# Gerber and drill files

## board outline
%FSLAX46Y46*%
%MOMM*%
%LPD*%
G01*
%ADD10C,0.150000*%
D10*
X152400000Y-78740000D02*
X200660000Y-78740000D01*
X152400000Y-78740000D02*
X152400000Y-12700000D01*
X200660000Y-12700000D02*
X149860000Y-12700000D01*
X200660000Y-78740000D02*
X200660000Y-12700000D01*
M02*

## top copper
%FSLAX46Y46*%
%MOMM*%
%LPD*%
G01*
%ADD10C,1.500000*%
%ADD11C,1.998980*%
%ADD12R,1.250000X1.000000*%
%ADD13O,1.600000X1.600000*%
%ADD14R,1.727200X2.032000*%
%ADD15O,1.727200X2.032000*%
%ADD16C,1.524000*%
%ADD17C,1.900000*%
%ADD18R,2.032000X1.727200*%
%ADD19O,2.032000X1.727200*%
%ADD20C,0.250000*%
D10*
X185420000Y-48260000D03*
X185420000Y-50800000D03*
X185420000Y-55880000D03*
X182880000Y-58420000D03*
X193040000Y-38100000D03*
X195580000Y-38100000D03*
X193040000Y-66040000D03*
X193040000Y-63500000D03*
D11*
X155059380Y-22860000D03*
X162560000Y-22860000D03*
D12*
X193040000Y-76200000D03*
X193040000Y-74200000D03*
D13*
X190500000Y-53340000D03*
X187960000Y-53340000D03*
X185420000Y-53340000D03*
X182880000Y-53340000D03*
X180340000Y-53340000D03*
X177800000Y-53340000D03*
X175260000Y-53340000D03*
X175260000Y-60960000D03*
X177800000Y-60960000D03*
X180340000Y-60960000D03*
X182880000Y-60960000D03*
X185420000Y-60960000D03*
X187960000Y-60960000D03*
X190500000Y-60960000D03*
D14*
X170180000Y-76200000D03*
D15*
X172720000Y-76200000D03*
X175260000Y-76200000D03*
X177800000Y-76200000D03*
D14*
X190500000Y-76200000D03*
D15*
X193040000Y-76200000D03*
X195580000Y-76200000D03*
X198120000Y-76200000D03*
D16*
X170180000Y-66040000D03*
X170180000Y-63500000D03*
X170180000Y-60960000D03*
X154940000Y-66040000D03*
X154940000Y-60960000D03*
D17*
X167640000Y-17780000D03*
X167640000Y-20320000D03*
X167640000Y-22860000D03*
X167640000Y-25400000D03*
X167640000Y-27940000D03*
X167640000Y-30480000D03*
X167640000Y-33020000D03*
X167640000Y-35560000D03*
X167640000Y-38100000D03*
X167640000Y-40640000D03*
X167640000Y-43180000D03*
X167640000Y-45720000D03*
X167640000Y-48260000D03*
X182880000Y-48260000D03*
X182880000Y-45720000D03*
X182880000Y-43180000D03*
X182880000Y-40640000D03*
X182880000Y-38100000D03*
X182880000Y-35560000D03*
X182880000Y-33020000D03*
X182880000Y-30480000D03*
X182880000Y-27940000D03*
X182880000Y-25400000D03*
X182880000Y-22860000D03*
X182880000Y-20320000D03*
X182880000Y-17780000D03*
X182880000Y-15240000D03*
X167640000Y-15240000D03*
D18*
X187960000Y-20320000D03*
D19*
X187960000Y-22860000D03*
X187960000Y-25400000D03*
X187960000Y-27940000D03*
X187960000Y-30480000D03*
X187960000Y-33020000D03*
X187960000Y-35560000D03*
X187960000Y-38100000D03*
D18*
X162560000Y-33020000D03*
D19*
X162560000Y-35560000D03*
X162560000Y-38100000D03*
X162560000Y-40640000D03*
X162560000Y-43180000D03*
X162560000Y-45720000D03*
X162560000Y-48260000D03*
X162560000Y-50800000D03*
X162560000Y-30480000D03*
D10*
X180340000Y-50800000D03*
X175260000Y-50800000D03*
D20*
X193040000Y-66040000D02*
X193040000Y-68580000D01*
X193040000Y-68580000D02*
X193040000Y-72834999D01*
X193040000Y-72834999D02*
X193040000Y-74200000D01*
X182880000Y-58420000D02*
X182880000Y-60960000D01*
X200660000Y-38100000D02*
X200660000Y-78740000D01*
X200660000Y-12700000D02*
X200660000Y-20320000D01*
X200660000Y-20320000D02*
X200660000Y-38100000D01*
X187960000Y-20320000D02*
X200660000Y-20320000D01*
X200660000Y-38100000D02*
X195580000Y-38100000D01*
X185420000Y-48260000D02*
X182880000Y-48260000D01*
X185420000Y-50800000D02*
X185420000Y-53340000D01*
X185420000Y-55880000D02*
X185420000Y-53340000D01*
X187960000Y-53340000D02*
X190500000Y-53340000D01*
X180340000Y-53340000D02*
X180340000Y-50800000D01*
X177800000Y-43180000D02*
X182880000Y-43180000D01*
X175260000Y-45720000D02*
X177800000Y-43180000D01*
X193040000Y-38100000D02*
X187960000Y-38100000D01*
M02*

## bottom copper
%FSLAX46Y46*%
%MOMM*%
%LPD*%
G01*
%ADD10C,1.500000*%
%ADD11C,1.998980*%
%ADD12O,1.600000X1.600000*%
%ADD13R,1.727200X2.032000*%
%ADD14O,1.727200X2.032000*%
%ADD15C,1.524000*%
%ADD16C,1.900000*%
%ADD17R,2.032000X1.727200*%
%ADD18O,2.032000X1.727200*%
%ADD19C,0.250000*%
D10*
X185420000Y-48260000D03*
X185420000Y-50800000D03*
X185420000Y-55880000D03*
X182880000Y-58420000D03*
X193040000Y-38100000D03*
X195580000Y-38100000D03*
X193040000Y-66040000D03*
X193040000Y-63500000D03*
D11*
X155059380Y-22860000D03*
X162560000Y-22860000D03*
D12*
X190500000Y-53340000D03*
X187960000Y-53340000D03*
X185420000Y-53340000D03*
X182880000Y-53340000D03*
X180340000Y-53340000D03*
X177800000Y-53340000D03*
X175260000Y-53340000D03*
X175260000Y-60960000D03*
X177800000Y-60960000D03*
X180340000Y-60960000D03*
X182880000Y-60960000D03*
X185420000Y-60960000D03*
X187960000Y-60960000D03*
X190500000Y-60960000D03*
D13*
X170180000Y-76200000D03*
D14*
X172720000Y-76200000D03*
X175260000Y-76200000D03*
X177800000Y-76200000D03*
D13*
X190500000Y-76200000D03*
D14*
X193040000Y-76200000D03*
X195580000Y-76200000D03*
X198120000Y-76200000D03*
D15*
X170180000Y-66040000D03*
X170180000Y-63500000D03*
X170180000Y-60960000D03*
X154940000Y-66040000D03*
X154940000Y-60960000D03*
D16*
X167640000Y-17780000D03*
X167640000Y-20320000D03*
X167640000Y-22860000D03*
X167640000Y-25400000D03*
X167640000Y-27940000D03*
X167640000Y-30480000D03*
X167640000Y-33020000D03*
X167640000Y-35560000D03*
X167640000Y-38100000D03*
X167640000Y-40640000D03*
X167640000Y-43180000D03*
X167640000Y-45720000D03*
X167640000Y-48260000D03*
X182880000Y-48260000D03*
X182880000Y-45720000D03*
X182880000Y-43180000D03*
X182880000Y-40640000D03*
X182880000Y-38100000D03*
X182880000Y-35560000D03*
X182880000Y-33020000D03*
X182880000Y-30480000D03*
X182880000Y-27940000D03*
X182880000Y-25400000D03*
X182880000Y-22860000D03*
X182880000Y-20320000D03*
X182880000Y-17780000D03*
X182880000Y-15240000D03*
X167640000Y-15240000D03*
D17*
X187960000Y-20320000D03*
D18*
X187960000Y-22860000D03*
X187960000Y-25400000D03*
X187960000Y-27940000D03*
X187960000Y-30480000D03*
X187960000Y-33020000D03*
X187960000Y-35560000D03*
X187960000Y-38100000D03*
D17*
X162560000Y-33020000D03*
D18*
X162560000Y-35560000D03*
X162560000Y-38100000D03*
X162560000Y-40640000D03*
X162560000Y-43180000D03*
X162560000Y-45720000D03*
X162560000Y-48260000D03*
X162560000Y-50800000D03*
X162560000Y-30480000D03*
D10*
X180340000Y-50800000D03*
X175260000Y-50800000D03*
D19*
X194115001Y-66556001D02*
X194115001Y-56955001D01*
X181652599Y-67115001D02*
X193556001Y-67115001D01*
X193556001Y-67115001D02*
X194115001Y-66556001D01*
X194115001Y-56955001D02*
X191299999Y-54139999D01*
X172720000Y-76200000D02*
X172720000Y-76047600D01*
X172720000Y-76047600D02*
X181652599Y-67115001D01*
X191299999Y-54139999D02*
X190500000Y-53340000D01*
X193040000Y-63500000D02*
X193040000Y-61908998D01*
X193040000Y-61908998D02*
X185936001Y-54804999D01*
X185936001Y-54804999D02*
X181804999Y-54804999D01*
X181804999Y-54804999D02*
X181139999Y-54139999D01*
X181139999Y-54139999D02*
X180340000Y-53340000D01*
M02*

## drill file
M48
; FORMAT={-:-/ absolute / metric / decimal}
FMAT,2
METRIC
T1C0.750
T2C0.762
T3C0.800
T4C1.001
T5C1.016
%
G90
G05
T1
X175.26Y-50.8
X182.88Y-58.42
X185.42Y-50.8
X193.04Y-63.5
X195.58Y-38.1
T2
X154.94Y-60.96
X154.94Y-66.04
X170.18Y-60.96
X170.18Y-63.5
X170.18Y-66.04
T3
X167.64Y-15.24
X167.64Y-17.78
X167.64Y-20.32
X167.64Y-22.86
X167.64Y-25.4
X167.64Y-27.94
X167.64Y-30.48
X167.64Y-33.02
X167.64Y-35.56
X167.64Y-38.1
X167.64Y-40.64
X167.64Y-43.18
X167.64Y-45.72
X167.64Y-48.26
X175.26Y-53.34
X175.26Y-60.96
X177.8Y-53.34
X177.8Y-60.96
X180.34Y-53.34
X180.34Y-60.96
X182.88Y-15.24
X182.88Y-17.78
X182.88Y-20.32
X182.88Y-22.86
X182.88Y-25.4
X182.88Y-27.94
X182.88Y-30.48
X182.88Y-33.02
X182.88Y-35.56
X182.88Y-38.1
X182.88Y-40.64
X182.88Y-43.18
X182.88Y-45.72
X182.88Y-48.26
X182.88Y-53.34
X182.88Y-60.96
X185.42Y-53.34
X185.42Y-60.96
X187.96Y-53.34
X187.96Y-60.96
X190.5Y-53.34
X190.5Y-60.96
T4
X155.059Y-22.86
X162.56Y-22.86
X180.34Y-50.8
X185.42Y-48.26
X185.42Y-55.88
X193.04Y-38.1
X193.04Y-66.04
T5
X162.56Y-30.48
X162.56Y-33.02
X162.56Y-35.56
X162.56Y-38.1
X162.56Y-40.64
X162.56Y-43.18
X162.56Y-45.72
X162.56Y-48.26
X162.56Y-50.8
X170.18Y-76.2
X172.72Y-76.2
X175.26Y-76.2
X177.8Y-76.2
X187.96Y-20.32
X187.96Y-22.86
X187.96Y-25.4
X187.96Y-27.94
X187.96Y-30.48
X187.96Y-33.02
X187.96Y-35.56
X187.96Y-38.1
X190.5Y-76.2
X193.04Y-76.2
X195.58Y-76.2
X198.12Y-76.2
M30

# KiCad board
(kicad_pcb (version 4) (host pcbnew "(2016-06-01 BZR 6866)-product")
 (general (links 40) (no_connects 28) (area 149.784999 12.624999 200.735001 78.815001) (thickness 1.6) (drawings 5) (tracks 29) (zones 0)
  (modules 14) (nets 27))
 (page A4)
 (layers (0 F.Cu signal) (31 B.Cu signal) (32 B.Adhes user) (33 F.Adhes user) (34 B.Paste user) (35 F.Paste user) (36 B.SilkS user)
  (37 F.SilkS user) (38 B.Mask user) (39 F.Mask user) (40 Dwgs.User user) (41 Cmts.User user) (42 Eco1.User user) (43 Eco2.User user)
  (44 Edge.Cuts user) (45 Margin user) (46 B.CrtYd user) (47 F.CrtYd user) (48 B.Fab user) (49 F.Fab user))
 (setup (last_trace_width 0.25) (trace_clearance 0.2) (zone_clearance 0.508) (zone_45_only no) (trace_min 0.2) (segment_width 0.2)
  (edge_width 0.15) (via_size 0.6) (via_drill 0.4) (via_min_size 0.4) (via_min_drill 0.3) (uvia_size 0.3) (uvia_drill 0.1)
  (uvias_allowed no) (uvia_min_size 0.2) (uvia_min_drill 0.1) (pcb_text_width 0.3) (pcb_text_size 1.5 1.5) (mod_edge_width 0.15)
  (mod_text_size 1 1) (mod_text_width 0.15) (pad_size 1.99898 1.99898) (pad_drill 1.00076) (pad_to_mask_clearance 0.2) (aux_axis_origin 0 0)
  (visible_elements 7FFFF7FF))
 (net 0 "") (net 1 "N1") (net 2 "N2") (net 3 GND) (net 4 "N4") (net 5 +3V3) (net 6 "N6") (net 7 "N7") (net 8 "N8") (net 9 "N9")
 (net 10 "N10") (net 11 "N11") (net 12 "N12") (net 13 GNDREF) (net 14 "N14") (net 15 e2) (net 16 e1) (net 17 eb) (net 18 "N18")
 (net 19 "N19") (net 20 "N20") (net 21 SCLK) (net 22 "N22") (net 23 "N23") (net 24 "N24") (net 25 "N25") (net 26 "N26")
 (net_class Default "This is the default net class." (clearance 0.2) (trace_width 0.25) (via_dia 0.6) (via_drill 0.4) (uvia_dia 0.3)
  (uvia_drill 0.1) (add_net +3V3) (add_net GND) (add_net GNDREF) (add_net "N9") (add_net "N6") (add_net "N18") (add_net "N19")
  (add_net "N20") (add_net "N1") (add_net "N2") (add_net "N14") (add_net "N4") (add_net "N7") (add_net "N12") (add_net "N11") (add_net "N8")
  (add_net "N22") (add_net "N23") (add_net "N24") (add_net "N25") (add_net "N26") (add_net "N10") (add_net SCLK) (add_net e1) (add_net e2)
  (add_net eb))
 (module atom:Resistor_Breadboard (layer F.Cu) (at 185.42 50.8 270)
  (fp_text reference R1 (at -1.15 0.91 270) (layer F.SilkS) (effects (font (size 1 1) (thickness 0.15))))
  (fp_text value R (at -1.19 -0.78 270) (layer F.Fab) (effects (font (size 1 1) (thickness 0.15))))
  (pad 1 thru_hole circle (at -2.54 0 270) (size 1.5 1.5) (drill 1.00076) (layers *.Cu *.SilkS *.Mask) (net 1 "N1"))
  (pad 2 thru_hole circle (at 0 0 270) (size 1.5 1.5) (drill 0.75) (layers *.Cu *.SilkS *.Mask) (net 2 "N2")))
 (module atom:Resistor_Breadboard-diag (layer F.Cu) (at 182.88 58.42 180)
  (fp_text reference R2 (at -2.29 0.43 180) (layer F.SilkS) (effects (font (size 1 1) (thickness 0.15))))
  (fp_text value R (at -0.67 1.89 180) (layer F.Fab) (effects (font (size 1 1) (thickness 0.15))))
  (pad 1 thru_hole circle (at -2.54 2.54 180) (size 1.5 1.5) (drill 1.00076) (layers *.Cu *.SilkS *.Mask) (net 2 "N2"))
  (pad 2 thru_hole circle (at 0 0 180) (size 1.5 1.5) (drill 0.75) (layers *.Cu *.SilkS *.Mask) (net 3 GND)))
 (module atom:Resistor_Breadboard (layer F.Cu) (at 195.58 38.1)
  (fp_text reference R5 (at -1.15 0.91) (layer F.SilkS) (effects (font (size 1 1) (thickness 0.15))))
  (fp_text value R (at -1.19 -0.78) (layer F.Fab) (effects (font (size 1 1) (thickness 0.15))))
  (pad 1 thru_hole circle (at -2.54 0) (size 1.5 1.5) (drill 1.00076) (layers *.Cu *.SilkS *.Mask) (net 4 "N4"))
  (pad 2 thru_hole circle (at 0 0) (size 1.5 1.5) (drill 0.75) (layers *.Cu *.SilkS *.Mask) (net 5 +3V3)))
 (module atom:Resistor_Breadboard (layer F.Cu) (at 193.04 63.5 90)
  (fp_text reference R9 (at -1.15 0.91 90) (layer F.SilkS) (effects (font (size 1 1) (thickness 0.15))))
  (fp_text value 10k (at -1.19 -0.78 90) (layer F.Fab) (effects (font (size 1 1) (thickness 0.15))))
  (pad 1 thru_hole circle (at -2.54 0 90) (size 1.5 1.5) (drill 1.00076) (layers *.Cu *.SilkS *.Mask) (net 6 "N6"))
  (pad 2 thru_hole circle (at 0 0 90) (size 1.5 1.5) (drill 0.75) (layers *.Cu *.SilkS *.Mask) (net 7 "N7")))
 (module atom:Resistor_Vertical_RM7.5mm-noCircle (layer F.Cu) (at 158.80842 22.86)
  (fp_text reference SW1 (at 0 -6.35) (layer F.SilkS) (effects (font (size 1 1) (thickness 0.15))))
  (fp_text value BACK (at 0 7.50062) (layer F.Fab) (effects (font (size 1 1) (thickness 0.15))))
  (pad 1 thru_hole circle (at -3.74904 0) (size 1.99898 1.99898) (drill 1.00076) (layers *.Cu *.SilkS *.Mask) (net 3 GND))
  (pad 2 thru_hole circle (at 3.75158 0) (size 1.99898 1.99898) (drill 1.00076) (layers *.Cu *.SilkS *.Mask) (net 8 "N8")))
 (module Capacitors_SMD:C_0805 (layer F.Cu) (at 193.04 75.2 90)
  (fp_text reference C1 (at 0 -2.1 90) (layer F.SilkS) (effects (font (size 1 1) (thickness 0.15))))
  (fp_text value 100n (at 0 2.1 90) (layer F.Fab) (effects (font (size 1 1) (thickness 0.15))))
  (pad 1 smd rect (at -1 0 90) (size 1 1.25) (layers F.Cu F.Paste F.Mask) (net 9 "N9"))
  (pad 2 smd rect (at 1 0 90) (size 1 1.25) (layers F.Cu F.Paste F.Mask) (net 6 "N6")))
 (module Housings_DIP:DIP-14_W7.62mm (layer F.Cu) (at 190.5 53.34 270)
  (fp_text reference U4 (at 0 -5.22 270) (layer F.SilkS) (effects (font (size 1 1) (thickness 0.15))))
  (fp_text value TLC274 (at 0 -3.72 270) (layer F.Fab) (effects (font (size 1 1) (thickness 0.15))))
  (pad 1 thru_hole oval (at 0 0 270) (size 1.6 1.6) (drill 0.8) (layers *.Cu *.Mask F.SilkS) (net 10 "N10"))
  (pad 2 thru_hole oval (at 0 2.54 270) (size 1.6 1.6) (drill 0.8) (layers *.Cu *.Mask F.SilkS) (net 10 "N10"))
  (pad 3 thru_hole oval (at 0 5.08 270) (size 1.6 1.6) (drill 0.8) (layers *.Cu *.Mask F.SilkS) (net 2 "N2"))
  (pad 4 thru_hole oval (at 0 7.62 270) (size 1.6 1.6) (drill 0.8) (layers *.Cu *.Mask F.SilkS) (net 5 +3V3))
  (pad 5 thru_hole oval (at 0 10.16 270) (size 1.6 1.6) (drill 0.8) (layers *.Cu *.Mask F.SilkS) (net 7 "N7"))
  (pad 6 thru_hole oval (at 0 12.7 270) (size 1.6 1.6) (drill 0.8) (layers *.Cu *.Mask F.SilkS) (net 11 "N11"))
  (pad 7 thru_hole oval (at 0 15.24 270) (size 1.6 1.6) (drill 0.8) (layers *.Cu *.Mask F.SilkS) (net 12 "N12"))
  (pad 8 thru_hole oval (at 7.62 15.24 270) (size 1.6 1.6) (drill 0.8) (layers *.Cu *.Mask F.SilkS) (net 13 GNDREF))
  (pad 9 thru_hole oval (at 7.62 12.7 270) (size 1.6 1.6) (drill 0.8) (layers *.Cu *.Mask F.SilkS) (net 13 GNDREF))
  (pad 10 thru_hole oval (at 7.62 10.16 270) (size 1.6 1.6) (drill 0.8) (layers *.Cu *.Mask F.SilkS) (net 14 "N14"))
  (pad 11 thru_hole oval (at 7.62 7.62 270) (size 1.6 1.6) (drill 0.8) (layers *.Cu *.Mask F.SilkS) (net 3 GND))
  (pad 12 thru_hole oval (at 7.62 5.08 270) (size 1.6 1.6) (drill 0.8) (layers *.Cu *.Mask F.SilkS))
  (pad 13 thru_hole oval (at 7.62 2.54 270) (size 1.6 1.6) (drill 0.8) (layers *.Cu *.Mask F.SilkS))
  (pad 14 thru_hole oval (at 7.62 0 270) (size 1.6 1.6) (drill 0.8) (layers *.Cu *.Mask F.SilkS)))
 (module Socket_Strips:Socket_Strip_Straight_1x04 (layer F.Cu) (at 170.18 76.2)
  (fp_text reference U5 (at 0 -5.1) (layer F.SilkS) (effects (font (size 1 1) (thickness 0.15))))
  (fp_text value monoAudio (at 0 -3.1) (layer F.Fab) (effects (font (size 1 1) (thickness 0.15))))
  (pad 1 thru_hole rect (at 0 0) (size 1.7272 2.032) (drill 1.016) (layers *.Cu *.Mask F.SilkS) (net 3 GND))
  (pad 2 thru_hole oval (at 2.54 0) (size 1.7272 2.032) (drill 1.016) (layers *.Cu *.Mask F.SilkS) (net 10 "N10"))
  (pad 3 thru_hole oval (at 5.08 0) (size 1.7272 2.032) (drill 1.016) (layers *.Cu *.Mask F.SilkS))
  (pad 4 thru_hole oval (at 7.62 0) (size 1.7272 2.032) (drill 1.016) (layers *.Cu *.Mask F.SilkS)))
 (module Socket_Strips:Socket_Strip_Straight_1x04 (layer F.Cu) (at 190.5 76.2)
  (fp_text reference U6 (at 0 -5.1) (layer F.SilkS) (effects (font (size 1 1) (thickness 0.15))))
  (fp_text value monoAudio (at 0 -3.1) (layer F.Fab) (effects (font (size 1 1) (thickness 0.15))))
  (pad 1 thru_hole rect (at 0 0) (size 1.7272 2.032) (drill 1.016) (layers *.Cu *.Mask F.SilkS) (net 3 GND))
  (pad 2 thru_hole oval (at 2.54 0) (size 1.7272 2.032) (drill 1.016) (layers *.Cu *.Mask F.SilkS) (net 9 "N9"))
  (pad 3 thru_hole oval (at 5.08 0) (size 1.7272 2.032) (drill 1.016) (layers *.Cu *.Mask F.SilkS))
  (pad 4 thru_hole oval (at 7.62 0) (size 1.7272 2.032) (drill 1.016) (layers *.Cu *.Mask F.SilkS)))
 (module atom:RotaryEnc (layer F.Cu) (at 162.56 63.5 180)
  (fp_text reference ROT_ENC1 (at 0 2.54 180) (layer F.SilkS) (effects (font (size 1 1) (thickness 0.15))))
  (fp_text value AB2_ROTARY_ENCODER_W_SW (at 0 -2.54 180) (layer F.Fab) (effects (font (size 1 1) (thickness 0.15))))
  (pad 1 thru_hole circle (at -7.62 -2.54 180) (size 1.524 1.524) (drill 0.762) (layers *.Cu *.Mask F.SilkS) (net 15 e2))
  (pad 2 thru_hole circle (at -7.62 0 180) (size 1.524 1.524) (drill 0.762) (layers *.Cu *.Mask F.SilkS) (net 3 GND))
  (pad 3 thru_hole circle (at -7.62 2.54 180) (size 1.524 1.524) (drill 0.762) (layers *.Cu *.Mask F.SilkS) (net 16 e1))
  (pad 4 thru_hole circle (at 7.62 -2.54 180) (size 1.524 1.524) (drill 0.762) (layers *.Cu *.Mask F.SilkS) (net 3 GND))
  (pad 5 thru_hole circle (at 7.62 2.54 180) (size 1.524 1.524) (drill 0.762) (layers *.Cu *.Mask F.SilkS) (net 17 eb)))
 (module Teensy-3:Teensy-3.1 (layer F.Cu) (at 167.64 17.78 270)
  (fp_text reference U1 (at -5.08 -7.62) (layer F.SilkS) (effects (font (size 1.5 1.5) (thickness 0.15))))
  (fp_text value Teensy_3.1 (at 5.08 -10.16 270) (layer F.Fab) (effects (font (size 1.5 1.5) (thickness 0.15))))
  (pad 0 thru_hole circle (at 0 0 270) (size 1.9 1.9) (drill 0.8) (layers *.Cu *.Mask F.SilkS))
  (pad 1 thru_hole circle (at 2.54 0 270) (size 1.9 1.9) (drill 0.8) (layers *.Cu *.Mask F.SilkS))
  (pad 2 thru_hole circle (at 5.08 0 270) (size 1.9 1.9) (drill 0.8) (layers *.Cu *.Mask F.SilkS) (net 8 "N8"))
  (pad 3 thru_hole circle (at 7.62 0 270) (size 1.9 1.9) (drill 0.8) (layers *.Cu *.Mask F.SilkS))
  (pad 4 thru_hole circle (at 10.16 0 270) (size 1.9 1.9) (drill 0.8) (layers *.Cu *.Mask F.SilkS))
  (pad 5 thru_hole circle (at 12.7 0 270) (size 1.9 1.9) (drill 0.8) (layers *.Cu *.Mask F.SilkS))
  (pad 6 thru_hole circle (at 15.24 0 270) (size 1.9 1.9) (drill 0.8) (layers *.Cu *.Mask F.SilkS) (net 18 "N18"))
  (pad 7 thru_hole circle (at 17.78 0 270) (size 1.9 1.9) (drill 0.8) (layers *.Cu *.Mask F.SilkS) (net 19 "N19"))
  (pad 8 thru_hole circle (at 20.32 0 270) (size 1.9 1.9) (drill 0.8) (layers *.Cu *.Mask F.SilkS))
  (pad 9 thru_hole circle (at 22.86 0 270) (size 1.9 1.9) (drill 0.8) (layers *.Cu *.Mask F.SilkS) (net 16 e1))
  (pad 10 thru_hole circle (at 25.4 0 270) (size 1.9 1.9) (drill 0.8) (layers *.Cu *.Mask F.SilkS) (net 15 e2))
  (pad 11 thru_hole circle (at 27.94 0 270) (size 1.9 1.9) (drill 0.8) (layers *.Cu *.Mask F.SilkS) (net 17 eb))
  (pad 12 thru_hole circle (at 30.48 0 270) (size 1.9 1.9) (drill 0.8) (layers *.Cu *.Mask F.SilkS) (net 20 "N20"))
  (pad 13 thru_hole circle (at 30.48 -15.24 270) (size 1.9 1.9) (drill 0.8) (layers *.Cu *.Mask F.SilkS) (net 1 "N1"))
  (pad 14 thru_hole circle (at 27.94 -15.24 270) (size 1.9 1.9) (drill 0.8) (layers *.Cu *.Mask F.SilkS) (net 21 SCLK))
  (pad 15 thru_hole circle (at 25.4 -15.24 270) (size 1.9 1.9) (drill 0.8) (layers *.Cu *.Mask F.SilkS) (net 12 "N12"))
  (pad 16 thru_hole circle (at 22.86 -15.24 270) (size 1.9 1.9) (drill 0.8) (layers *.Cu *.Mask F.SilkS))
  (pad 17 thru_hole circle (at 20.32 -15.24 270) (size 1.9 1.9) (drill 0.8) (layers *.Cu *.Mask F.SilkS))
  (pad 18 thru_hole circle (at 17.78 -15.24 270) (size 1.9 1.9) (drill 0.8) (layers *.Cu *.Mask F.SilkS) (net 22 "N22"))
  (pad 19 thru_hole circle (at 15.24 -15.24 270) (size 1.9 1.9) (drill 0.8) (layers *.Cu *.Mask F.SilkS) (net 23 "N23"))
  (pad 20 thru_hole circle (at 12.7 -15.24 270) (size 1.9 1.9) (drill 0.8) (layers *.Cu *.Mask F.SilkS) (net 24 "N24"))
  (pad 21 thru_hole circle (at 10.16 -15.24 270) (size 1.9 1.9) (drill 0.8) (layers *.Cu *.Mask F.SilkS) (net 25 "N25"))
  (pad 22 thru_hole circle (at 7.62 -15.24 270) (size 1.9 1.9) (drill 0.8) (layers *.Cu *.Mask F.SilkS) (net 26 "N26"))
  (pad 23 thru_hole circle (at 5.08 -15.24 270) (size 1.9 1.9) (drill 0.8) (layers *.Cu *.Mask F.SilkS))
  (pad 24 thru_hole circle (at 2.54 -15.24 270) (size 1.9 1.9) (drill 0.8) (layers *.Cu *.Mask F.SilkS) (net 5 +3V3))
  (pad 25 thru_hole circle (at 0 -15.24 270) (size 1.9 1.9) (drill 0.8) (layers *.Cu *.Mask F.SilkS))
  (pad 26 thru_hole circle (at -2.54 -15.24 270) (size 1.9 1.9) (drill 0.8) (layers *.Cu *.Mask F.SilkS))
  (pad 27 thru_hole circle (at -2.54 0 270) (size 1.9 1.9) (drill 0.8) (layers *.Cu *.Mask F.SilkS) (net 3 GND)))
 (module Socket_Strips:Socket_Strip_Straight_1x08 (layer F.Cu) (at 187.96 20.32 270)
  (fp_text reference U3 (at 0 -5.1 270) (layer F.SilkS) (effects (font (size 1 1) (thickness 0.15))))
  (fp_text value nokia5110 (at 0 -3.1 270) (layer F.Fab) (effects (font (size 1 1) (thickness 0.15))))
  (pad 1 thru_hole rect (at 0 0 270) (size 1.7272 2.032) (drill 1.016) (layers *.Cu *.Mask F.SilkS) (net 5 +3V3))
  (pad 2 thru_hole oval (at 2.54 0 270) (size 1.7272 2.032) (drill 1.016) (layers *.Cu *.Mask F.SilkS) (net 3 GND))
  (pad 3 thru_hole oval (at 5.08 0 270) (size 1.7272 2.032) (drill 1.016) (layers *.Cu *.Mask F.SilkS) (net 26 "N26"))
  (pad 4 thru_hole oval (at 7.62 0 270) (size 1.7272 2.032) (drill 1.016) (layers *.Cu *.Mask F.SilkS) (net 25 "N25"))
  (pad 5 thru_hole oval (at 10.16 0 270) (size 1.7272 2.032) (drill 1.016) (layers *.Cu *.Mask F.SilkS) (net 24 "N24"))
  (pad 6 thru_hole oval (at 12.7 0 270) (size 1.7272 2.032) (drill 1.016) (layers *.Cu *.Mask F.SilkS) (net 23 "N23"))
  (pad 7 thru_hole oval (at 15.24 0 270) (size 1.7272 2.032) (drill 1.016) (layers *.Cu *.Mask F.SilkS) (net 22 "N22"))
  (pad 8 thru_hole oval (at 17.78 0 270) (size 1.7272 2.032) (drill 1.016) (layers *.Cu *.Mask F.SilkS) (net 4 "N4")))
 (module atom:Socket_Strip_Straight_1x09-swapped (layer F.Cu) (at 162.56 33.02 270)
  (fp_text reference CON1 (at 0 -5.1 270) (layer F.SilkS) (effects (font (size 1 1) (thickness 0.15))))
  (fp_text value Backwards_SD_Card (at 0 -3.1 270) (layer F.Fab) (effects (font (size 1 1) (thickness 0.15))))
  (pad 1 thru_hole rect (at 0 0 270) (size 1.7272 2.032) (drill 1.016) (layers *.Cu *.Mask F.SilkS) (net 18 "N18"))
  (pad 2 thru_hole oval (at 2.54 0 270) (size 1.7272 2.032) (drill 1.016) (layers *.Cu *.Mask F.SilkS) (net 19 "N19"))
  (pad 3 thru_hole oval (at 5.08 0 270) (size 1.7272 2.032) (drill 1.016) (layers *.Cu *.Mask F.SilkS) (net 3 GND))
  (pad 4 thru_hole oval (at 7.62 0 270) (size 1.7272 2.032) (drill 1.016) (layers *.Cu *.Mask F.SilkS) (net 5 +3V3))
  (pad 5 thru_hole oval (at 10.16 0 270) (size 1.7272 2.032) (drill 1.016) (layers *.Cu *.Mask F.SilkS) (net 21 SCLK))
  (pad 6 thru_hole oval (at 12.7 0 270) (size 1.7272 2.032) (drill 1.016) (layers *.Cu *.Mask F.SilkS) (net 3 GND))
  (pad 7 thru_hole oval (at 15.24 0 270) (size 1.7272 2.032) (drill 1.016) (layers *.Cu *.Mask F.SilkS) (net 20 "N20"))
  (pad 8 thru_hole oval (at 17.78 0 270) (size 1.7272 2.032) (drill 1.016) (layers *.Cu *.Mask F.SilkS))
  (pad 9 thru_hole oval (at -2.54 0 270) (size 1.7272 2.032) (drill 1.016) (layers *.Cu *.Mask F.SilkS)))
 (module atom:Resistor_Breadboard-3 (layer F.Cu) (at 177.8 50.8 180)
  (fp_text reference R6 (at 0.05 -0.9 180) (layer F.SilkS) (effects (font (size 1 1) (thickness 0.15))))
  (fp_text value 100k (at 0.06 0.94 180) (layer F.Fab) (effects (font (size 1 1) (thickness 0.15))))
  (pad 1 thru_hole circle (at -2.54 0 180) (size 1.5 1.5) (drill 1.00076) (layers *.Cu *.SilkS *.Mask) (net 7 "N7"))
  (pad 2 thru_hole circle (at 2.54 0 180) (size 1.5 1.5) (drill 0.75) (layers *.Cu *.SilkS *.Mask) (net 12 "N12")))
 (gr_line (start 152.4 78.74) (end 200.66 78.74) (layer Edge.Cuts) (width 0.15))
 (gr_line (start 152.4 78.74) (end 152.4 12.7) (layer Edge.Cuts) (width 0.15))
 (gr_line (start 200.66 12.7) (end 149.86 12.7) (layer Edge.Cuts) (width 0.15))
 (gr_line (start 200.66 78.74) (end 200.66 12.7) (layer Edge.Cuts) (width 0.15))
 (segment (start 193.04 66.04) (end 193.04 68.58) (width 0.25) (layer F.Cu) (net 6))
 (segment (start 193.04 68.58) (end 193.04 72.834999) (width 0.25) (layer F.Cu) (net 6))
 (segment (start 193.04 72.834999) (end 193.04 74.2) (width 0.25) (layer F.Cu) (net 6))
 (segment (start 182.88 58.42) (end 182.88 60.96) (width 0.25) (layer F.Cu) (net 3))
 (segment (start 200.66 38.1) (end 200.66 78.74) (width 0.25) (layer F.Cu) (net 5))
 (segment (start 200.66 12.7) (end 200.66 20.32) (width 0.25) (layer F.Cu) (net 5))
 (segment (start 200.66 20.32) (end 200.66 38.1) (width 0.25) (layer F.Cu) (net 5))
 (segment (start 187.96 20.32) (end 200.66 20.32) (width 0.25) (layer F.Cu) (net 5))
 (segment (start 200.66 38.1) (end 195.58 38.1) (width 0.25) (layer F.Cu) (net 5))
 (segment (start 185.42 48.26) (end 182.88 48.26) (width 0.25) (layer F.Cu) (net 1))
 (segment (start 185.42 50.8) (end 185.42 53.34) (width 0.25) (layer F.Cu) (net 2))
 (segment (start 185.42 55.88) (end 185.42 53.34) (width 0.25) (layer F.Cu) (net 2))
 (segment (start 194.115001 66.556001) (end 194.115001 56.955001) (width 0.25) (layer B.Cu) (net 10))
 (segment (start 181.652599 67.115001) (end 193.556001 67.115001) (width 0.25) (layer B.Cu) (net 10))
 (segment (start 193.556001 67.115001) (end 194.115001 66.556001) (width 0.25) (layer B.Cu) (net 10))
 (segment (start 194.115001 56.955001) (end 191.299999 54.139999) (width 0.25) (layer B.Cu) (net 10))
 (segment (start 187.96 53.34) (end 190.5 53.34) (width 0.25) (layer F.Cu) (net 10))
 (segment (start 172.72 76.2) (end 172.72 76.0476) (width 0.25) (layer B.Cu) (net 10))
 (segment (start 172.72 76.0476) (end 181.652599 67.115001) (width 0.25) (layer B.Cu) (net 10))
 (segment (start 191.299999 54.139999) (end 190.5 53.34) (width 0.25) (layer B.Cu) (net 10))
 (segment (start 193.04 63.5) (end 193.04 61.908998) (width 0.25) (layer B.Cu) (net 7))
 (segment (start 193.04 61.908998) (end 185.936001 54.804999) (width 0.25) (layer B.Cu) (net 7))
 (segment (start 185.936001 54.804999) (end 181.804999 54.804999) (width 0.25) (layer B.Cu) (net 7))
 (segment (start 181.804999 54.804999) (end 181.139999 54.139999) (width 0.25) (layer B.Cu) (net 7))
 (segment (start 181.139999 54.139999) (end 180.34 53.34) (width 0.25) (layer B.Cu) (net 7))
 (segment (start 180.34 53.34) (end 180.34 50.8) (width 0.25) (layer F.Cu) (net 7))
 (segment (start 177.8 43.18) (end 182.88 43.18) (width 0.25) (layer F.Cu) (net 12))
 (segment (start 175.26 45.72) (end 177.8 43.18) (width 0.25) (layer F.Cu) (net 12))
 (segment (start 193.04 38.1) (end 187.96 38.1) (width 0.25) (layer F.Cu) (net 4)))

